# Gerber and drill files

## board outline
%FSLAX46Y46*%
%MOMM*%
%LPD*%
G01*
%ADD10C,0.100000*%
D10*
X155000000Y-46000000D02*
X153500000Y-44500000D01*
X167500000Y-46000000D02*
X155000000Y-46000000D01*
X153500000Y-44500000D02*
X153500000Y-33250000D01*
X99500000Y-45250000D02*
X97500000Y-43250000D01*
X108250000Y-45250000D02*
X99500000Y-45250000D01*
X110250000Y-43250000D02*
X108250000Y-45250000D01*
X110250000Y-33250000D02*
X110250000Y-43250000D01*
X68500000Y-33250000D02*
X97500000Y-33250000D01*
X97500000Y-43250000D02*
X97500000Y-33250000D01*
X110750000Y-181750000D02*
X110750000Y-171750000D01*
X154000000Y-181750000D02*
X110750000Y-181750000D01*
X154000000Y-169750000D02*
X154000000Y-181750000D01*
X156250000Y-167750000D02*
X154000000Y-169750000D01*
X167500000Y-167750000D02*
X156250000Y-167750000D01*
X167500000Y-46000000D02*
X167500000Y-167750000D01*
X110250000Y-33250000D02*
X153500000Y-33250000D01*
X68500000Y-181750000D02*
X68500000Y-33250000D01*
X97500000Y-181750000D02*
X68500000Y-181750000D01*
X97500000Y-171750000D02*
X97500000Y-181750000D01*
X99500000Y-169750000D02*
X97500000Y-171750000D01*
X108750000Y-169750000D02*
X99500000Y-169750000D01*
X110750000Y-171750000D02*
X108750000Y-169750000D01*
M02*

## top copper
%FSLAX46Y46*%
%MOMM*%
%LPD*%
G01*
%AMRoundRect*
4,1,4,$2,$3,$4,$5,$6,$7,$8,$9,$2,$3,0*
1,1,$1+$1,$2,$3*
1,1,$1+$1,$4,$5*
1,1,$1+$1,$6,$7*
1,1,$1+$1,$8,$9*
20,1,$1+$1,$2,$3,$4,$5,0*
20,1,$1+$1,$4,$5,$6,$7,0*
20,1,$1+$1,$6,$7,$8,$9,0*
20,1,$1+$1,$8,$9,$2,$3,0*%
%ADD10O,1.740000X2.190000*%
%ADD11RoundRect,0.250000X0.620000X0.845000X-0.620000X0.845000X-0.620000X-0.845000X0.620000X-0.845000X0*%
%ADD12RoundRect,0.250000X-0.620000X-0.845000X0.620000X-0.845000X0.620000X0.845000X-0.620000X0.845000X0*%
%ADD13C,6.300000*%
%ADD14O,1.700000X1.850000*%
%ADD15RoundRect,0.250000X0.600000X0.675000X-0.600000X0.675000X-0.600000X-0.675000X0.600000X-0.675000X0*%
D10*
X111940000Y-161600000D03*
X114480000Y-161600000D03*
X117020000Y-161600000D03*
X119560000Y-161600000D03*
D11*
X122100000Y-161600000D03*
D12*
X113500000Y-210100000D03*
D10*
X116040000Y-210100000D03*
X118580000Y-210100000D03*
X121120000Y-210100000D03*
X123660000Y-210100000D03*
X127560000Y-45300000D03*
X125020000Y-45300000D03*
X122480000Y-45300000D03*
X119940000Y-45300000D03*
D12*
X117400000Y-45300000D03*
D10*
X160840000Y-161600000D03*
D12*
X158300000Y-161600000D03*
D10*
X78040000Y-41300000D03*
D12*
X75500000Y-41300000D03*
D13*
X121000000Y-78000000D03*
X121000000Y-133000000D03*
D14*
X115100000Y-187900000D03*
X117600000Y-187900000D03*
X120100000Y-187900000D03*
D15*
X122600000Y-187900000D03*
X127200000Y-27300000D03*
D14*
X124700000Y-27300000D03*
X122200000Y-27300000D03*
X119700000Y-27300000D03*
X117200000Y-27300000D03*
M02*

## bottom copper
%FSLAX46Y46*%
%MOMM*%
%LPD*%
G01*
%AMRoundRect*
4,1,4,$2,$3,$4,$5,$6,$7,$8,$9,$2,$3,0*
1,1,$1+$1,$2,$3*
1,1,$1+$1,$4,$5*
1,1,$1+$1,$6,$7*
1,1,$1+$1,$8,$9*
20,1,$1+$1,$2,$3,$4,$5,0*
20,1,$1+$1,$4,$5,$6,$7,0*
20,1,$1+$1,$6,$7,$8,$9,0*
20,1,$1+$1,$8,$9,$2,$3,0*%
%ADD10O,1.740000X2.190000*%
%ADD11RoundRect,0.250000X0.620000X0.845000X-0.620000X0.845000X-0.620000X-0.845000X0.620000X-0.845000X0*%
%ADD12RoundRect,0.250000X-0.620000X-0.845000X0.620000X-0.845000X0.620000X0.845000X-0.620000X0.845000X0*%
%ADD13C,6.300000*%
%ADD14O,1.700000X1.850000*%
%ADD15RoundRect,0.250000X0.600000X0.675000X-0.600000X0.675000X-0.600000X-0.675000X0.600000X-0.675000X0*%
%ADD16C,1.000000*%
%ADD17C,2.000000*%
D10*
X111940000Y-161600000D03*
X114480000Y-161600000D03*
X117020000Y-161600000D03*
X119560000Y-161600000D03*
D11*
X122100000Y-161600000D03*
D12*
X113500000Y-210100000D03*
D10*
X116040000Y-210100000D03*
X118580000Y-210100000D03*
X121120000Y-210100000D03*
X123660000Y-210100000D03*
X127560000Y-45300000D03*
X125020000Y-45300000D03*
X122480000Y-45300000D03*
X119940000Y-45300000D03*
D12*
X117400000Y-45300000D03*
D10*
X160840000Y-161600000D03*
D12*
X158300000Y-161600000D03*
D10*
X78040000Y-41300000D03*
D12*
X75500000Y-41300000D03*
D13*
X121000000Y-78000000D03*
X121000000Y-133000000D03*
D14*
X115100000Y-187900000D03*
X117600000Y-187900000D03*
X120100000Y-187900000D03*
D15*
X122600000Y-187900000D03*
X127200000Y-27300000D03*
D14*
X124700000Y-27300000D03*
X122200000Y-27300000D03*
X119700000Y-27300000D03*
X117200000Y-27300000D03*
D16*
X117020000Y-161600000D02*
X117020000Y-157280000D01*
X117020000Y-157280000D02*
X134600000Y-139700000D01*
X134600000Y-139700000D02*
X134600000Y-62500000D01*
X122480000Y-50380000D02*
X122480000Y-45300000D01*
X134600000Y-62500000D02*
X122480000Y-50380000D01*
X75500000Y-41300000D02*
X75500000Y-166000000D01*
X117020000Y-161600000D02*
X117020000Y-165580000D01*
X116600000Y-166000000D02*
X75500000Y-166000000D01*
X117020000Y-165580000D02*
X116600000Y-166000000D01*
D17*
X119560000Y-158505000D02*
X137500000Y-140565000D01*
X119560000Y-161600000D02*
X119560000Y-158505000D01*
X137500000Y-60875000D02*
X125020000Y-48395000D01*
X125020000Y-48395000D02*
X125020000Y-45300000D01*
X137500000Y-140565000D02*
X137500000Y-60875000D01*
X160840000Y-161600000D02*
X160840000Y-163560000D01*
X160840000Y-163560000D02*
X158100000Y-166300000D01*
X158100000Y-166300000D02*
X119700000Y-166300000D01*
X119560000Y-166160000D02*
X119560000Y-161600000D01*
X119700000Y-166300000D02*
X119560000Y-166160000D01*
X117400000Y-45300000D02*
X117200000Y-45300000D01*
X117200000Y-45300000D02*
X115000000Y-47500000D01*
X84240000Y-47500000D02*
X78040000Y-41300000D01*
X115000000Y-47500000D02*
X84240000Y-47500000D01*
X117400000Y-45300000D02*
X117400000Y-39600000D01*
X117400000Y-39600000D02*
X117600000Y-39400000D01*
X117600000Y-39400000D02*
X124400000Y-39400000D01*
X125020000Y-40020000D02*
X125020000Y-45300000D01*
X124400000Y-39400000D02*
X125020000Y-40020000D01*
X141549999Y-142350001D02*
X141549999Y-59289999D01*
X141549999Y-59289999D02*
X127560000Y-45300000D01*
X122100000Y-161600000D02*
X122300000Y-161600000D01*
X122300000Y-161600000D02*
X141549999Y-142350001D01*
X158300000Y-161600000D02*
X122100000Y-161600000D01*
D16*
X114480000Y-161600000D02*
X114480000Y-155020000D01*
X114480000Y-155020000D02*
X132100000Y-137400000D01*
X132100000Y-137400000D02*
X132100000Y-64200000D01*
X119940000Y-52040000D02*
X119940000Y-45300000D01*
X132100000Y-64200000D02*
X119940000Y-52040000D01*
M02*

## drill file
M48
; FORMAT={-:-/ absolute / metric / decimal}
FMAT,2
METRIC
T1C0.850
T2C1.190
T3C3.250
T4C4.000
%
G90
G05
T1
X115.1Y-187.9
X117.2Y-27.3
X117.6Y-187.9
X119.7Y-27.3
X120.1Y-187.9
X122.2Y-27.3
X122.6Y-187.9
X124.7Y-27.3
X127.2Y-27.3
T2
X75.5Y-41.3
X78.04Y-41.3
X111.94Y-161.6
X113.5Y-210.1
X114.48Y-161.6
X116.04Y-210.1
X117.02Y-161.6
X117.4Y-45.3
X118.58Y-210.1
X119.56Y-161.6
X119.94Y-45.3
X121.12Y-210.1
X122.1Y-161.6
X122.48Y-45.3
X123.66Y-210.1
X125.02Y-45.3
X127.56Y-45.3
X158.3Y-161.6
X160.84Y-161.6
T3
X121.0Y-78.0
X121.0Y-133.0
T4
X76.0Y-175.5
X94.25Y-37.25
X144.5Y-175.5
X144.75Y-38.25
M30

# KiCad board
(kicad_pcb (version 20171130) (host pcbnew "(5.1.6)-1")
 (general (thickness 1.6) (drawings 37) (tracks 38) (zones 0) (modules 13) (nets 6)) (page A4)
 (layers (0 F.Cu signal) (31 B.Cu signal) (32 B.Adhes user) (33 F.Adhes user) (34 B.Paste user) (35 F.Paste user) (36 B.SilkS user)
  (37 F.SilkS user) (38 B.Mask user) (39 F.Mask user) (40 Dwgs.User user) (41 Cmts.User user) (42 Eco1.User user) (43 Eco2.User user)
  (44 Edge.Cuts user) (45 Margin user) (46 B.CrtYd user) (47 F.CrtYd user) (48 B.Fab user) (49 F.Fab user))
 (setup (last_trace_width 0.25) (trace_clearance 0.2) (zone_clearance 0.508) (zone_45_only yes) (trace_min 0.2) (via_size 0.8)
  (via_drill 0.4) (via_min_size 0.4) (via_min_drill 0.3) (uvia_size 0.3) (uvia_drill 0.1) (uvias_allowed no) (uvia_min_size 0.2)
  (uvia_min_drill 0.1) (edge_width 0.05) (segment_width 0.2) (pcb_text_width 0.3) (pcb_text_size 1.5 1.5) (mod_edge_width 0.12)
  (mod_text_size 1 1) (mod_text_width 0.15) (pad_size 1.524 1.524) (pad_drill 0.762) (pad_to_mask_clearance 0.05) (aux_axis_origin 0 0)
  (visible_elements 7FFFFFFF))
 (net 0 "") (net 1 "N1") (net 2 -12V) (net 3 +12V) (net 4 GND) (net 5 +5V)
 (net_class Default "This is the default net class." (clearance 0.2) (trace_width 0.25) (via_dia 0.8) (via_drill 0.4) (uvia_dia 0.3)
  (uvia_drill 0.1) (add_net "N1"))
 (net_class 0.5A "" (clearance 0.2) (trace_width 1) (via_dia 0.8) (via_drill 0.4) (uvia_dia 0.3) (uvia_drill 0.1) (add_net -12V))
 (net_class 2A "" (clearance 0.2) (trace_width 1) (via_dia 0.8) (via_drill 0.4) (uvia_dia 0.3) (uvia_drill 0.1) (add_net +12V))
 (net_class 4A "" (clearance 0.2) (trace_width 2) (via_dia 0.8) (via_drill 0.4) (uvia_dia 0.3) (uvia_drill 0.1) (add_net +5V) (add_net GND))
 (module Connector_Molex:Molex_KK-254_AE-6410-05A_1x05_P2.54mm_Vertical (layer F.Cu) (at 122.1 161.6 180)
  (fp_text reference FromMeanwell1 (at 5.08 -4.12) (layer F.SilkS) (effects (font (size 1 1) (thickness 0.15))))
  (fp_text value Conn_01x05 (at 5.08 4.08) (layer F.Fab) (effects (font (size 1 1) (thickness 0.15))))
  (pad 5 thru_hole oval (at 10.16 0 180) (size 1.74 2.19) (drill 1.19) (layers *.Cu *.Mask) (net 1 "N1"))
  (pad 4 thru_hole oval (at 7.62 0 180) (size 1.74 2.19) (drill 1.19) (layers *.Cu *.Mask) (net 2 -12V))
  (pad 3 thru_hole oval (at 5.08 0 180) (size 1.74 2.19) (drill 1.19) (layers *.Cu *.Mask) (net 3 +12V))
  (pad 2 thru_hole oval (at 2.54 0 180) (size 1.74 2.19) (drill 1.19) (layers *.Cu *.Mask) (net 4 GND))
  (pad 1 thru_hole roundrect (at 0 0 180) (size 1.74 2.19) (drill 1.19) (layers *.Cu *.Mask) (roundrect_rratio 0.143678) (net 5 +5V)))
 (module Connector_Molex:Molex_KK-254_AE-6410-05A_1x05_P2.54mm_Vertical (layer F.Cu) (at 113.5 210.1)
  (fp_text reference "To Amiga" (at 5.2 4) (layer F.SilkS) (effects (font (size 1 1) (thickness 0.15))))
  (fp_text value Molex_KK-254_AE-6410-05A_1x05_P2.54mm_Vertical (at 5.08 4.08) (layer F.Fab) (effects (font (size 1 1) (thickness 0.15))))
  (pad 1 thru_hole roundrect (at 0 0) (size 1.74 2.19) (drill 1.19) (layers *.Cu *.Mask) (roundrect_rratio 0.143678))
  (pad 2 thru_hole oval (at 2.54 0) (size 1.74 2.19) (drill 1.19) (layers *.Cu *.Mask))
  (pad 3 thru_hole oval (at 5.08 0) (size 1.74 2.19) (drill 1.19) (layers *.Cu *.Mask))
  (pad 4 thru_hole oval (at 7.62 0) (size 1.74 2.19) (drill 1.19) (layers *.Cu *.Mask))
  (pad 5 thru_hole oval (at 10.16 0) (size 1.74 2.19) (drill 1.19) (layers *.Cu *.Mask)))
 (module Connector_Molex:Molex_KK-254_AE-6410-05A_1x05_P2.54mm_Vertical (layer F.Cu) (at 117.4 45.3)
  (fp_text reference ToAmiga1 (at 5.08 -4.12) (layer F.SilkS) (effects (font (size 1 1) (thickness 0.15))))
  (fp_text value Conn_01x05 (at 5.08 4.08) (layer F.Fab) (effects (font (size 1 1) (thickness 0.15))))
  (pad 5 thru_hole oval (at 10.16 0) (size 1.74 2.19) (drill 1.19) (layers *.Cu *.Mask) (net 5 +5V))
  (pad 4 thru_hole oval (at 7.62 0) (size 1.74 2.19) (drill 1.19) (layers *.Cu *.Mask) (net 4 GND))
  (pad 3 thru_hole oval (at 5.08 0) (size 1.74 2.19) (drill 1.19) (layers *.Cu *.Mask) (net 3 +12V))
  (pad 2 thru_hole oval (at 2.54 0) (size 1.74 2.19) (drill 1.19) (layers *.Cu *.Mask) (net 2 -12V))
  (pad 1 thru_hole roundrect (at 0 0) (size 1.74 2.19) (drill 1.19) (layers *.Cu *.Mask) (roundrect_rratio 0.143678) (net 4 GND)))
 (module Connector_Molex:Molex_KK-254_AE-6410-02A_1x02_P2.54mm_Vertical (layer F.Cu) (at 158.3 161.6)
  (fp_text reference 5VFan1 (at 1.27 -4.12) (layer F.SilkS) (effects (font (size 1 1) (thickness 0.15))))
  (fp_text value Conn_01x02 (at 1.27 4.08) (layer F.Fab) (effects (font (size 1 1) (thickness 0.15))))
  (pad 2 thru_hole oval (at 2.54 0) (size 1.74 2.19) (drill 1.19) (layers *.Cu *.Mask) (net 4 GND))
  (pad 1 thru_hole roundrect (at 0 0) (size 1.74 2.19) (drill 1.19) (layers *.Cu *.Mask) (roundrect_rratio 0.143678) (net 5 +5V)))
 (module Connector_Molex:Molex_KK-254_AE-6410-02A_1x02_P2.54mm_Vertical (layer F.Cu) (at 75.5 41.3)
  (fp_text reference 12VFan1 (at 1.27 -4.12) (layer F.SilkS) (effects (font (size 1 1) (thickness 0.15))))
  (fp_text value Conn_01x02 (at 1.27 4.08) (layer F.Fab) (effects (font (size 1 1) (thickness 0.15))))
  (pad 2 thru_hole oval (at 2.54 0) (size 1.74 2.19) (drill 1.19) (layers *.Cu *.Mask) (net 4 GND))
  (pad 1 thru_hole roundrect (at 0 0) (size 1.74 2.19) (drill 1.19) (layers *.Cu *.Mask) (roundrect_rratio 0.143678) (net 3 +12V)))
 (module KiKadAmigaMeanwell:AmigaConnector (layer F.Cu) (at 84 69.25)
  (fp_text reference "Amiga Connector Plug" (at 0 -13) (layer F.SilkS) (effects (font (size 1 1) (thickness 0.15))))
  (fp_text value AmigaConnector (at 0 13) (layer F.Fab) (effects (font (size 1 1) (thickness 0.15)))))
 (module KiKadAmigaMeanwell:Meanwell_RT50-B (layer F.Cu) (at 111.5 104.5 90)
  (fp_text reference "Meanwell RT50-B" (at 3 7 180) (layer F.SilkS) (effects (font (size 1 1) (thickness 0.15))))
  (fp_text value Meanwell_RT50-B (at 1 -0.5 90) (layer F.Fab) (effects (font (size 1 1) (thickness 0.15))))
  (pad "" np_thru_hole circle (at 26.5 9.5 90) (size 6.3 6.3) (drill 3.25) (layers *.Cu *.Mask))
  (pad "" np_thru_hole circle (at -28.5 9.5 90) (size 6.3 6.3) (drill 3.25) (layers *.Cu *.Mask)))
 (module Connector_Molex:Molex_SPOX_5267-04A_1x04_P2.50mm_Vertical (layer F.Cu) (at 122.6 187.9 180)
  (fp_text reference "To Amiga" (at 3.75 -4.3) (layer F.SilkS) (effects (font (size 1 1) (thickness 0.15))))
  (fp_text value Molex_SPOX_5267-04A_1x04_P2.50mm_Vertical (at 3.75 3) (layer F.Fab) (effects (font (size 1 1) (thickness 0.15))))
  (pad 4 thru_hole oval (at 7.5 0 180) (size 1.7 1.85) (drill 0.85) (layers *.Cu *.Mask))
  (pad 3 thru_hole oval (at 5 0 180) (size 1.7 1.85) (drill 0.85) (layers *.Cu *.Mask))
  (pad 2 thru_hole oval (at 2.5 0 180) (size 1.7 1.85) (drill 0.85) (layers *.Cu *.Mask))
  (pad 1 thru_hole roundrect (at 0 0 180) (size 1.7 1.85) (drill 0.85) (layers *.Cu *.Mask) (roundrect_rratio 0.147059)))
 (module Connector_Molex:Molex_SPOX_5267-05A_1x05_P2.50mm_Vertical (layer F.Cu) (at 127.2 27.3 180)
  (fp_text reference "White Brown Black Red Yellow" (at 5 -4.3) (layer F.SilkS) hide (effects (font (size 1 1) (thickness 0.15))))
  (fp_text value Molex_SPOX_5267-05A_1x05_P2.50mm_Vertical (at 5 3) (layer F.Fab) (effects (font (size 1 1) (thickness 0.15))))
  (pad 1 thru_hole roundrect (at 0 0 180) (size 1.7 1.85) (drill 0.85) (layers *.Cu *.Mask) (roundrect_rratio 0.147059))
  (pad 2 thru_hole oval (at 2.5 0 180) (size 1.7 1.85) (drill 0.85) (layers *.Cu *.Mask))
  (pad 3 thru_hole oval (at 5 0 180) (size 1.7 1.85) (drill 0.85) (layers *.Cu *.Mask))
  (pad 4 thru_hole oval (at 7.5 0 180) (size 1.7 1.85) (drill 0.85) (layers *.Cu *.Mask))
  (pad 5 thru_hole oval (at 10 0 180) (size 1.7 1.85) (drill 0.85) (layers *.Cu *.Mask)))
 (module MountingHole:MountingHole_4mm (layer F.Cu) (at 94.25 37.25 180)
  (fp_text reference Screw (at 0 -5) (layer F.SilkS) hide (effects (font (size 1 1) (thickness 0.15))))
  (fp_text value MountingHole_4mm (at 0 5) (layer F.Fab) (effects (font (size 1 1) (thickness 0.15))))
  (pad 1 np_thru_hole circle (at 0 0 180) (size 4 4) (drill 4) (layers *.Cu *.Mask)))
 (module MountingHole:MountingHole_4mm (layer F.Cu) (at 144.75 38.25 180)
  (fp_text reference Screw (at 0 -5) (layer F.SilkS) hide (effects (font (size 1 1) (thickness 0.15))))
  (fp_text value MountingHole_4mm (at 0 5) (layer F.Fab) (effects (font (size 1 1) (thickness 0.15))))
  (pad 1 np_thru_hole circle (at 0 0 180) (size 4 4) (drill 4) (layers *.Cu *.Mask)))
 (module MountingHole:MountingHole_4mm (layer F.Cu) (at 144.5 175.5 180)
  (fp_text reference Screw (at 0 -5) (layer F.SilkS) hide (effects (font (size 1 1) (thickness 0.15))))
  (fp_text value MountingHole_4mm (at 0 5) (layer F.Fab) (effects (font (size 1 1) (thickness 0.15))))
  (pad 1 np_thru_hole circle (at 0 0 180) (size 4 4) (drill 4) (layers *.Cu *.Mask)))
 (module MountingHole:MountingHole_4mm (layer F.Cu) (at 76 175.5 180)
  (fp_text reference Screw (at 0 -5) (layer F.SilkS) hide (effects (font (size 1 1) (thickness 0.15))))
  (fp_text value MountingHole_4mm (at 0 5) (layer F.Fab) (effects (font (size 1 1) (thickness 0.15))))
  (pad 1 np_thru_hole circle (at 0 0 180) (size 4 4) (drill 4) (layers *.Cu *.Mask)))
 (gr_line (start 155 46) (end 153.5 44.5) (layer Edge.Cuts) (width 0.1))
 (gr_line (start 167.5 46) (end 155 46) (layer Edge.Cuts) (width 0.1))
 (gr_line (start 153.5 44.5) (end 153.5 33.25) (layer Edge.Cuts) (width 0.1))
 (gr_line (start 99.5 45.25) (end 97.5 43.25) (layer Edge.Cuts) (width 0.1))
 (gr_line (start 108.25 45.25) (end 99.5 45.25) (layer Edge.Cuts) (width 0.1))
 (gr_line (start 110.25 43.25) (end 108.25 45.25) (layer Edge.Cuts) (width 0.1))
 (gr_line (start 110.25 33.25) (end 110.25 43.25) (layer Edge.Cuts) (width 0.1))
 (gr_line (start 68.5 33.25) (end 97.5 33.25) (layer Edge.Cuts) (width 0.1))
 (gr_line (start 97.5 43.25) (end 97.5 33.25) (layer Edge.Cuts) (width 0.1))
 (gr_line (start 110.75 181.75) (end 110.75 171.75) (layer Edge.Cuts) (width 0.1))
 (gr_line (start 154 181.75) (end 110.75 181.75) (layer Edge.Cuts) (width 0.1))
 (gr_line (start 154 169.75) (end 154 181.75) (layer Edge.Cuts) (width 0.1))
 (gr_line (start 156.25 167.75) (end 154 169.75) (layer Edge.Cuts) (width 0.1))
 (gr_line (start 167.5 167.75) (end 156.25 167.75) (layer Edge.Cuts) (width 0.1))
 (gr_line (start 167.5 46) (end 167.5 167.75) (layer Edge.Cuts) (width 0.1))
 (gr_line (start 110.25 33.25) (end 153.5 33.25) (layer Edge.Cuts) (width 0.1))
 (gr_line (start 68.5 181.75) (end 68.5 33.25) (layer Edge.Cuts) (width 0.1))
 (gr_line (start 97.5 181.75) (end 68.5 181.75) (layer Edge.Cuts) (width 0.1))
 (gr_line (start 97.5 171.75) (end 97.5 181.75) (layer Edge.Cuts) (width 0.1))
 (gr_line (start 99.5 169.75) (end 97.5 171.75) (layer Edge.Cuts) (width 0.1))
 (gr_line (start 108.75 169.75) (end 99.5 169.75) (layer Edge.Cuts) (width 0.1))
 (gr_line (start 110.75 171.75) (end 108.75 169.75) (layer Edge.Cuts) (width 0.1))
 (segment (start 117.02 161.6) (end 117.02 157.28) (width 1) (layer B.Cu) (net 3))
 (segment (start 117.02 157.28) (end 134.6 139.7) (width 1) (layer B.Cu) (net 3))
 (segment (start 134.6 139.7) (end 134.6 62.5) (width 1) (layer B.Cu) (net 3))
 (segment (start 122.48 50.38) (end 122.48 45.3) (width 1) (layer B.Cu) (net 3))
 (segment (start 134.6 62.5) (end 122.48 50.38) (width 1) (layer B.Cu) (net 3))
 (segment (start 75.5 41.3) (end 75.5 166) (width 1) (layer B.Cu) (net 3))
 (segment (start 117.02 161.6) (end 117.02 165.58) (width 1) (layer B.Cu) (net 3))
 (segment (start 116.6 166) (end 75.5 166) (width 1) (layer B.Cu) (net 3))
 (segment (start 117.02 165.58) (end 116.6 166) (width 1) (layer B.Cu) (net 3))
 (segment (start 119.56 158.505) (end 137.5 140.565) (width 2) (layer B.Cu) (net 4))
 (segment (start 119.56 161.6) (end 119.56 158.505) (width 2) (layer B.Cu) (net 4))
 (segment (start 137.5 60.875) (end 125.02 48.395) (width 2) (layer B.Cu) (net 4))
 (segment (start 125.02 48.395) (end 125.02 45.3) (width 2) (layer B.Cu) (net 4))
 (segment (start 137.5 140.565) (end 137.5 60.875) (width 2) (layer B.Cu) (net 4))
 (segment (start 160.84 161.6) (end 160.84 163.56) (width 2) (layer B.Cu) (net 4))
 (segment (start 160.84 163.56) (end 158.1 166.3) (width 2) (layer B.Cu) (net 4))
 (segment (start 158.1 166.3) (end 119.7 166.3) (width 2) (layer B.Cu) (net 4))
 (segment (start 119.56 166.16) (end 119.56 161.6) (width 2) (layer B.Cu) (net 4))
 (segment (start 119.7 166.3) (end 119.56 166.16) (width 2) (layer B.Cu) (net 4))
 (segment (start 117.4 45.3) (end 117.2 45.3) (width 2) (layer B.Cu) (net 4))
 (segment (start 117.2 45.3) (end 115 47.5) (width 2) (layer B.Cu) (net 4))
 (segment (start 84.24 47.5) (end 78.04 41.3) (width 2) (layer B.Cu) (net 4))
 (segment (start 115 47.5) (end 84.24 47.5) (width 2) (layer B.Cu) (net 4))
 (segment (start 117.4 45.3) (end 117.4 39.6) (width 2) (layer B.Cu) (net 4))
 (segment (start 117.4 39.6) (end 117.6 39.4) (width 2) (layer B.Cu) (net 4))
 (segment (start 117.6 39.4) (end 124.4 39.4) (width 2) (layer B.Cu) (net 4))
 (segment (start 125.02 40.02) (end 125.02 45.3) (width 2) (layer B.Cu) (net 4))
 (segment (start 124.4 39.4) (end 125.02 40.02) (width 2) (layer B.Cu) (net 4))
 (segment (start 141.549999 142.350001) (end 141.549999 59.289999) (width 2) (layer B.Cu) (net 5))
 (segment (start 141.549999 59.289999) (end 127.56 45.3) (width 2) (layer B.Cu) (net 5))
 (segment (start 122.1 161.6) (end 122.3 161.6) (width 2) (layer B.Cu) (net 5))
 (segment (start 122.3 161.6) (end 141.549999 142.350001) (width 2) (layer B.Cu) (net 5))
 (segment (start 158.3 161.6) (end 122.1 161.6) (width 2) (layer B.Cu) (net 5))
 (segment (start 114.48 161.6) (end 114.48 155.02) (width 1) (layer B.Cu) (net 2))
 (segment (start 114.48 155.02) (end 132.1 137.4) (width 1) (layer B.Cu) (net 2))
 (segment (start 132.1 137.4) (end 132.1 64.2) (width 1) (layer B.Cu) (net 2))
 (segment (start 119.94 52.04) (end 119.94 45.3) (width 1) (layer B.Cu) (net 2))
 (segment (start 132.1 64.2) (end 119.94 52.04) (width 1) (layer B.Cu) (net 2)))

